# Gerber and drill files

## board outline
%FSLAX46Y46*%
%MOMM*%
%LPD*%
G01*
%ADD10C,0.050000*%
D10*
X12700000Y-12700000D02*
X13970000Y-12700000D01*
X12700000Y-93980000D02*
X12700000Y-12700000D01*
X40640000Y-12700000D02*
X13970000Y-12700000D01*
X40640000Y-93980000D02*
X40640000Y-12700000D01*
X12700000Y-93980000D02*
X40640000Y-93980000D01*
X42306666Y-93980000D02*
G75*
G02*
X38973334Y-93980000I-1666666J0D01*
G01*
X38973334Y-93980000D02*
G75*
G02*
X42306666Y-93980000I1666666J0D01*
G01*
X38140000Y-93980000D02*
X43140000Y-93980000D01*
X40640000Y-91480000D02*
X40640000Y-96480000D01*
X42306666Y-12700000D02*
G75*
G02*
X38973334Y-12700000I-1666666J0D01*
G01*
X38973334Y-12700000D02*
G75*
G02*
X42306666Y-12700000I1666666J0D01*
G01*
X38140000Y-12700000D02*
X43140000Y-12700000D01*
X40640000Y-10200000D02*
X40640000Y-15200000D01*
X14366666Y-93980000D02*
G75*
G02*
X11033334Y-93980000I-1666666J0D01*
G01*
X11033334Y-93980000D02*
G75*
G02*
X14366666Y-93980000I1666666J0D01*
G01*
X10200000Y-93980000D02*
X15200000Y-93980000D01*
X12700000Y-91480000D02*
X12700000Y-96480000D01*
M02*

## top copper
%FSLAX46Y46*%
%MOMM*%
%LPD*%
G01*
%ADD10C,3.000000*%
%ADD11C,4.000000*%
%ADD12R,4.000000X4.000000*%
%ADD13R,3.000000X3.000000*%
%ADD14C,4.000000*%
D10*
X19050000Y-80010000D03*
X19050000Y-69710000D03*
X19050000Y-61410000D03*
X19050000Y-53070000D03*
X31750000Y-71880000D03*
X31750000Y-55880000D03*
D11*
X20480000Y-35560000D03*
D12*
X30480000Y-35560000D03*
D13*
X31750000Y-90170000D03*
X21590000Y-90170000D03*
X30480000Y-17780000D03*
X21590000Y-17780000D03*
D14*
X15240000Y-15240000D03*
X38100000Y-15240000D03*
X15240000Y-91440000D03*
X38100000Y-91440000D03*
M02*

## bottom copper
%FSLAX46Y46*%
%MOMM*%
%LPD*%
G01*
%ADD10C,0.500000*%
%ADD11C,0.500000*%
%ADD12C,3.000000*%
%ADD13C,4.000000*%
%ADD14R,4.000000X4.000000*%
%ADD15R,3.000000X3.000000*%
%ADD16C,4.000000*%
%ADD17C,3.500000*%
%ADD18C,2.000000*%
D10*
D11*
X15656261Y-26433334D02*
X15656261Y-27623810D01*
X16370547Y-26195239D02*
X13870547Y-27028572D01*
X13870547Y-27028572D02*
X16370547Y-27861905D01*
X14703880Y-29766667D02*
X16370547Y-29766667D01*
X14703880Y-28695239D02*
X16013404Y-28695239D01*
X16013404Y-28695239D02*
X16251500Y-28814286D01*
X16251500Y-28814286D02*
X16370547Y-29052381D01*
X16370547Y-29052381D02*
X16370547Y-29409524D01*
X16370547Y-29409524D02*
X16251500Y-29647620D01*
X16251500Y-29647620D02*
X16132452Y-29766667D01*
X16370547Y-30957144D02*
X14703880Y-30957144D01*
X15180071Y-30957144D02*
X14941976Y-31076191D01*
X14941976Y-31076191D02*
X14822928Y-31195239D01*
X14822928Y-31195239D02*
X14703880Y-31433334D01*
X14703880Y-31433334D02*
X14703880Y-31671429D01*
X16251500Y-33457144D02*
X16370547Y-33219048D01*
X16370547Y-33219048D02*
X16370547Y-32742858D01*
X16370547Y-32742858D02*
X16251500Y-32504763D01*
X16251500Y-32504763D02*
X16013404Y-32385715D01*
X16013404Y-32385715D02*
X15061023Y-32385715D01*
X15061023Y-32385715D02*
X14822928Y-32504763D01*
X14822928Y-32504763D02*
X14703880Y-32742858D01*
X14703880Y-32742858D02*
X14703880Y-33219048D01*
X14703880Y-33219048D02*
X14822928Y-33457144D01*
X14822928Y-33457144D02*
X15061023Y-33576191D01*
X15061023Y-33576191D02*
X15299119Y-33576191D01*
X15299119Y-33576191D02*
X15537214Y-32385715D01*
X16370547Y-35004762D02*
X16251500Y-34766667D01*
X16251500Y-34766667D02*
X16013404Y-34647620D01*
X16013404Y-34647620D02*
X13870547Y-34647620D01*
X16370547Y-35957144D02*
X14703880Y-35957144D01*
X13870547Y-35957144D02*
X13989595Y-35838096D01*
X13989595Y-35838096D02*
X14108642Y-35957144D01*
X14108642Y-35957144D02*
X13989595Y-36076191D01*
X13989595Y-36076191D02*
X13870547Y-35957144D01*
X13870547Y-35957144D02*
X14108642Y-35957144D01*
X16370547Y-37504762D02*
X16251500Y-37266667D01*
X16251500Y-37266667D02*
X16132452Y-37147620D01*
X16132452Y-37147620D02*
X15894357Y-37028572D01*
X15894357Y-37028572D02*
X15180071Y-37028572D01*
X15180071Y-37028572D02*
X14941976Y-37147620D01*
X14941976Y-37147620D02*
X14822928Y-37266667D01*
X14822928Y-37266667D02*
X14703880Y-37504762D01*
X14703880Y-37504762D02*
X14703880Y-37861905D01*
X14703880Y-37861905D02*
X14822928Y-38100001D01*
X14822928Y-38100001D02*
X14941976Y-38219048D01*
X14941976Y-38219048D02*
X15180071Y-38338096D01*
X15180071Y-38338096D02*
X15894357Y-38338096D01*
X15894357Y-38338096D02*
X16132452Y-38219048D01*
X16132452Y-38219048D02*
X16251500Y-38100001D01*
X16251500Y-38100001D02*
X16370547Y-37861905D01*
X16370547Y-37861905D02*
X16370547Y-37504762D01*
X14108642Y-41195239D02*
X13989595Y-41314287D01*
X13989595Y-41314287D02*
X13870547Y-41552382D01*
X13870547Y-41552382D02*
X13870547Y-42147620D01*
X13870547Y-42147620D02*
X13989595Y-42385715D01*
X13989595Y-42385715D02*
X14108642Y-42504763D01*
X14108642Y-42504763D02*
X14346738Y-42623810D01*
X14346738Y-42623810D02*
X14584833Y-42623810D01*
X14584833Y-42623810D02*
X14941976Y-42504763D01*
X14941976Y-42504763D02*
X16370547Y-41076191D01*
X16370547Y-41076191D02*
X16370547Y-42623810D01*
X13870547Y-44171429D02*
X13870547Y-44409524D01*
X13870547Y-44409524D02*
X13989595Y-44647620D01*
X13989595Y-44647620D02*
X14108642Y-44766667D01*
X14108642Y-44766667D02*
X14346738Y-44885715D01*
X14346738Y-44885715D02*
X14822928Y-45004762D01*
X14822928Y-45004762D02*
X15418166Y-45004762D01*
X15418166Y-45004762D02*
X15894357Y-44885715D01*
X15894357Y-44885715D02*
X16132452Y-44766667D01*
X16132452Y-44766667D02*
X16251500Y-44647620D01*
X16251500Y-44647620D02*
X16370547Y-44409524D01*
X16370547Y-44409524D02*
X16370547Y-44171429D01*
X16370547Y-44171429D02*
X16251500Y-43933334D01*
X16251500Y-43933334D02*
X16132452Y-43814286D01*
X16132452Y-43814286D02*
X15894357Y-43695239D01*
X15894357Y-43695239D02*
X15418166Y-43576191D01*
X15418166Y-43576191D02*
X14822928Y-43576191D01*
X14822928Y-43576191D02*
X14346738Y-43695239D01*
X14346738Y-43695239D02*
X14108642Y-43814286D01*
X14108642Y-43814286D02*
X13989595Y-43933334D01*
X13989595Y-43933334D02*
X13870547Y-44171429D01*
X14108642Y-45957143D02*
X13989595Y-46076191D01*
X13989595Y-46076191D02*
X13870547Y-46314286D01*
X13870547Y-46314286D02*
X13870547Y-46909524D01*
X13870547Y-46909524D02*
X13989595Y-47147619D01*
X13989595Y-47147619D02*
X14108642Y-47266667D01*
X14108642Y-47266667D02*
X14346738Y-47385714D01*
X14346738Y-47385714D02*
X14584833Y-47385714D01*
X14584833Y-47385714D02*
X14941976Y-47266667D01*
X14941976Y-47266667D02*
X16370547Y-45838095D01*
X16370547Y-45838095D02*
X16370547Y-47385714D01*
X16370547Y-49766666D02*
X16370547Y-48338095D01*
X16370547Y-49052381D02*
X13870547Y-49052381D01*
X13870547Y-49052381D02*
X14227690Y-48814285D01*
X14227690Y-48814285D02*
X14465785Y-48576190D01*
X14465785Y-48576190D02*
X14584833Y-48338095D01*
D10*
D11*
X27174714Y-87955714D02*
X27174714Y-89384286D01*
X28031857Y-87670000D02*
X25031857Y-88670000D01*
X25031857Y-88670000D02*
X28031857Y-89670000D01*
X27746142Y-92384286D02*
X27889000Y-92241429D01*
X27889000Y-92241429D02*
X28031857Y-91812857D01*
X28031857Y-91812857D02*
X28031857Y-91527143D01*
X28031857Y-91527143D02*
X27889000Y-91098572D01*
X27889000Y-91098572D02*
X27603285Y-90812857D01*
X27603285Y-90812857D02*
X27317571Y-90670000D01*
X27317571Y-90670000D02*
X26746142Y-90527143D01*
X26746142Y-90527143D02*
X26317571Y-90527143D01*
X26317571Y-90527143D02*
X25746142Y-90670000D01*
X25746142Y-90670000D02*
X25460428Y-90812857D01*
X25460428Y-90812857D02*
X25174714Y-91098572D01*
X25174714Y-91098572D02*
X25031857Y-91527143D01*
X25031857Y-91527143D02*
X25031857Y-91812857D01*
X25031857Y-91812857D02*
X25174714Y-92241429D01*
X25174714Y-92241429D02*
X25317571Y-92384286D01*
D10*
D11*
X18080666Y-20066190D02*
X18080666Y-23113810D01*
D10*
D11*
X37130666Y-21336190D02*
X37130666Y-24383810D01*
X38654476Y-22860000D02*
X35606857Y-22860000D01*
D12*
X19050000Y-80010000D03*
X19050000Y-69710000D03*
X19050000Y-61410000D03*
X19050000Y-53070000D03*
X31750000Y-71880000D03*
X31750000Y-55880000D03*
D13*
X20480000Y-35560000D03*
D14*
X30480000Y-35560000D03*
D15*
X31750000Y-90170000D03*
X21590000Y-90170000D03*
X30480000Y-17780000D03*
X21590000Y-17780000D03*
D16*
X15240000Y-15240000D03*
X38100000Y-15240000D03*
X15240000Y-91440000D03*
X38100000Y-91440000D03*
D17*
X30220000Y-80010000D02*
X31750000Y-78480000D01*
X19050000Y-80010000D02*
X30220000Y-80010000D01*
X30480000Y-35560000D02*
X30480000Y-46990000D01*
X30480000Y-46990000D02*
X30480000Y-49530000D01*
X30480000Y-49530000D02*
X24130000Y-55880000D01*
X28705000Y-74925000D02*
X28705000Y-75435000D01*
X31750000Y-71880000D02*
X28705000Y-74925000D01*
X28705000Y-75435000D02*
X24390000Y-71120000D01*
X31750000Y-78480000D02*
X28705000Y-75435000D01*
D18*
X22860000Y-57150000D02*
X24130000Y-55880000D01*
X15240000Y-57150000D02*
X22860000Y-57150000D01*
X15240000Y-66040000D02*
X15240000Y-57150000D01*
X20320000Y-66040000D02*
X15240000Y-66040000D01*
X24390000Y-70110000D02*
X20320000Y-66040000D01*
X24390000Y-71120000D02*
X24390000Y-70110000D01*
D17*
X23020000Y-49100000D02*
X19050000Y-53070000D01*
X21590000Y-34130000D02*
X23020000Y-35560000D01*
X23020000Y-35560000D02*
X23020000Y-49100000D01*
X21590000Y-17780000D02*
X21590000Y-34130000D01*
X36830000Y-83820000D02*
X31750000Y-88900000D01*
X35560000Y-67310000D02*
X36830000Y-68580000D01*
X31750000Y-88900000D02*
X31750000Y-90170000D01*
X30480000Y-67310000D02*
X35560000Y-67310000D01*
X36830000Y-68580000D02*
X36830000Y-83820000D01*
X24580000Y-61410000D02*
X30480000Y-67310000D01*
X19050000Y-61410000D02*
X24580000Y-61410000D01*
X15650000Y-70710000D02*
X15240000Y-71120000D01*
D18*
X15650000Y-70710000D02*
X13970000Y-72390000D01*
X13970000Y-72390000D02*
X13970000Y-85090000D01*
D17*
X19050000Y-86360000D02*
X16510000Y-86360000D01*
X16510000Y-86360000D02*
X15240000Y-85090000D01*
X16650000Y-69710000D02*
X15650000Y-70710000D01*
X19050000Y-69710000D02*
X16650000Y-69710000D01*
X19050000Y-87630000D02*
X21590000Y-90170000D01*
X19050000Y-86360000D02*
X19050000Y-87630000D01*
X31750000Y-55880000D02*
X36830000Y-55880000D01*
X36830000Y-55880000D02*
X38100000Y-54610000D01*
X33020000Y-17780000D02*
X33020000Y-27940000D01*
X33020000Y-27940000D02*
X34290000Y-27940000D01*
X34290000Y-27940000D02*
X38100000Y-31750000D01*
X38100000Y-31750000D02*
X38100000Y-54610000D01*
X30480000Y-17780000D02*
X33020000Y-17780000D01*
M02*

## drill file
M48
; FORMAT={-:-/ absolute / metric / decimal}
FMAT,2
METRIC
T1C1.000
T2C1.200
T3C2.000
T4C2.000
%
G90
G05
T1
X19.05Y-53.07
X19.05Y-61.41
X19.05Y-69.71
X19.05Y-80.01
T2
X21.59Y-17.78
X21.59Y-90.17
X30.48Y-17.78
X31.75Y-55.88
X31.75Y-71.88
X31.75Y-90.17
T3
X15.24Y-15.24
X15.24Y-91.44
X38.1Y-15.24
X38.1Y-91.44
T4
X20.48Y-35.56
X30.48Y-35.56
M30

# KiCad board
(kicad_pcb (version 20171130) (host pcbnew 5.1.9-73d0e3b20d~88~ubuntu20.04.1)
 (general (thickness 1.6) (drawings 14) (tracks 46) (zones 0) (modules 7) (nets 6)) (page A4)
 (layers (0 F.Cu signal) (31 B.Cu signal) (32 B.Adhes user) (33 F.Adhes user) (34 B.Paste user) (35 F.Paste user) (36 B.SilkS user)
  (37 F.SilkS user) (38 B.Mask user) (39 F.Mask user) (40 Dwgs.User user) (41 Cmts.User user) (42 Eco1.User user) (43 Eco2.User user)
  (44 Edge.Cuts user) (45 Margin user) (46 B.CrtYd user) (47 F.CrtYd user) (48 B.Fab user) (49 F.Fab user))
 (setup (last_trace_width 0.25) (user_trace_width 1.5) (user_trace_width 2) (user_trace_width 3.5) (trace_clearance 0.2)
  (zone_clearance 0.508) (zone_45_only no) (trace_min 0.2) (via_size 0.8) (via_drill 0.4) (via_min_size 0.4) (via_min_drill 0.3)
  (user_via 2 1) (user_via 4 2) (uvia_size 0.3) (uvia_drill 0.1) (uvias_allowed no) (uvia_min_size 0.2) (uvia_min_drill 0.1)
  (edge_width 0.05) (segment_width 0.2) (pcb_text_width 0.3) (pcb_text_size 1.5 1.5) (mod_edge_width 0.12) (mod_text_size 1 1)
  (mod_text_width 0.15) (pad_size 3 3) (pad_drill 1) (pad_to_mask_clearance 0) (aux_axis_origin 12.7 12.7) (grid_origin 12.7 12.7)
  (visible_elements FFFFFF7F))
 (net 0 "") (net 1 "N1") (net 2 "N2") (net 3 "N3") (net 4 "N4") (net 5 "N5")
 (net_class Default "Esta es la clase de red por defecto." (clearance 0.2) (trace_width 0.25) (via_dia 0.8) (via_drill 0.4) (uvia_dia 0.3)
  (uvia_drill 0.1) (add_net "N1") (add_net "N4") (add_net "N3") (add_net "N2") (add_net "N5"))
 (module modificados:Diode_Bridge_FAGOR (layer F.Cu) (at 19.05 78.74 90)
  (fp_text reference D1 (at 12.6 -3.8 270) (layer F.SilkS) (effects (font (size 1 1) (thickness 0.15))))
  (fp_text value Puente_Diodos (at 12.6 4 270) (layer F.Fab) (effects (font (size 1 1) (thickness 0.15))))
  (pad 1 thru_hole circle (at -1.27 0 90) (size 3 3) (drill 1) (layers *.Cu *.Mask) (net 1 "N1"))
  (pad 4 thru_hole circle (at 9.03 0 90) (size 3 3) (drill 1) (layers *.Cu *.Mask) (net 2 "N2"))
  (pad 3 thru_hole circle (at 17.33 0 90) (size 3 3) (drill 1) (layers *.Cu *.Mask) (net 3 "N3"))
  (pad 2 thru_hole circle (at 25.67 0 90) (size 3 3) (drill 1) (layers *.Cu *.Mask) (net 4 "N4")))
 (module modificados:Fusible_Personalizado (layer F.Cu) (at 31.75 55.88 270)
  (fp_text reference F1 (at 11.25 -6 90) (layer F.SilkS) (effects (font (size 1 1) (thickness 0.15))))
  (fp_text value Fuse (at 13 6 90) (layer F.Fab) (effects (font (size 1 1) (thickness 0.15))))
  (pad 2 thru_hole circle (at 16 0 270) (size 3 3) (drill 1.2) (layers *.Cu *.Mask) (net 1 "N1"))
  (pad 1 thru_hole circle (at 0 0 270) (size 3 3) (drill 1.2) (layers *.Cu *.Mask) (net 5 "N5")))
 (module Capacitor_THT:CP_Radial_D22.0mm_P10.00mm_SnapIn (layer F.Cu) (at 30.48 35.56 180)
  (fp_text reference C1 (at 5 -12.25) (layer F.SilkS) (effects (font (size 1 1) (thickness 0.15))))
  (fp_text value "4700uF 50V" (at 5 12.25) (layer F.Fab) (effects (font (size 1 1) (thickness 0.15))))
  (pad 2 thru_hole circle (at 10 0 180) (size 4 4) (drill 2) (layers *.Cu *.Mask) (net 4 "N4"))
  (pad 1 thru_hole rect (at 0 0 180) (size 4 4) (drill 2) (layers *.Cu *.Mask) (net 1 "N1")))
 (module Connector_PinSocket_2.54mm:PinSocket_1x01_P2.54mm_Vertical (layer F.Cu) (at 31.75 90.17 90)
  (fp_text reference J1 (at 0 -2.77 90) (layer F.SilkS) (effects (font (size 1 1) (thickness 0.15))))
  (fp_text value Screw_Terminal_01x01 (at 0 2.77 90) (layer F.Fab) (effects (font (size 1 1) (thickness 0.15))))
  (pad 1 thru_hole rect (at 0 0 90) (size 3 3) (drill 1.2) (layers *.Cu *.Mask) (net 3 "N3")))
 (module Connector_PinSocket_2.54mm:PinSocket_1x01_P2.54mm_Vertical (layer F.Cu) (at 21.59 90.17 90)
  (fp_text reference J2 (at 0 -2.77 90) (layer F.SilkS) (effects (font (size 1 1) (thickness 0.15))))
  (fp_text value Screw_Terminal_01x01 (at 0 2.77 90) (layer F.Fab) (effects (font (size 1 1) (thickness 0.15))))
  (pad 1 thru_hole rect (at 0 0 90) (size 3 3) (drill 1.2) (layers *.Cu *.Mask) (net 2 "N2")))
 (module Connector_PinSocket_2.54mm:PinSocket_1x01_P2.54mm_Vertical (layer F.Cu) (at 30.48 17.78 90)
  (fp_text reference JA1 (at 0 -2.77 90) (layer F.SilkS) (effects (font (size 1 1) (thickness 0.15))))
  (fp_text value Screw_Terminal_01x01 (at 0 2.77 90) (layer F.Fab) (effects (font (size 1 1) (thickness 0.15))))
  (pad 1 thru_hole rect (at 0 0 90) (size 3 3) (drill 1.2) (layers *.Cu *.Mask) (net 5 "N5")))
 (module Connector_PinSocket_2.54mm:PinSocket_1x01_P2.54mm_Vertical (layer F.Cu) (at 21.59 17.78 90)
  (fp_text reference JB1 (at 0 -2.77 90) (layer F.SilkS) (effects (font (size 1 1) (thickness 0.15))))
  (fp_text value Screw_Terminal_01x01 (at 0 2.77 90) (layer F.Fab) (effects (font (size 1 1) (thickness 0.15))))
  (pad 1 thru_hole rect (at 0 0 90) (size 3 3) (drill 1.2) (layers *.Cu *.Mask) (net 4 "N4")))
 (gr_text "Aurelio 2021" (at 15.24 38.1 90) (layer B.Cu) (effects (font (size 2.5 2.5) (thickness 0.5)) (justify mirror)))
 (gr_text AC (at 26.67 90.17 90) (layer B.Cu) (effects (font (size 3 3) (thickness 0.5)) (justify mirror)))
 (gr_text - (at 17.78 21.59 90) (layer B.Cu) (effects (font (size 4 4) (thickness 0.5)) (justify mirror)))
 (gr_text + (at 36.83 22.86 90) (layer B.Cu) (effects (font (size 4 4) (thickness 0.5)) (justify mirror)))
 (gr_line (start 12.7 12.7) (end 13.97 12.7) (layer Edge.Cuts) (width 0.05))
 (gr_line (start 12.7 93.98) (end 12.7 12.7) (layer Edge.Cuts) (width 0.05))
 (gr_line (start 40.64 12.7) (end 13.97 12.7) (layer Edge.Cuts) (width 0.05))
 (gr_line (start 40.64 93.98) (end 40.64 12.7) (layer Edge.Cuts) (width 0.05))
 (gr_line (start 12.7 93.98) (end 40.64 93.98) (layer Edge.Cuts) (width 0.05))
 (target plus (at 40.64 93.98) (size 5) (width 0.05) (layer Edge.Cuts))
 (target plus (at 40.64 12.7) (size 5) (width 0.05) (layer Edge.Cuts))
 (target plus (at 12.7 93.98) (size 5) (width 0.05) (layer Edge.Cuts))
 (via (at 15.24 15.24) (size 4) (drill 2) (layers F.Cu B.Cu) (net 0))
 (via (at 38.1 15.24) (size 4) (drill 2) (layers F.Cu B.Cu) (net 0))
 (via (at 15.24 91.44) (size 4) (drill 2) (layers F.Cu B.Cu) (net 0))
 (via (at 38.1 91.44) (size 4) (drill 2) (layers F.Cu B.Cu) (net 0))
 (segment (start 30.22 80.01) (end 31.75 78.48) (width 3.5) (layer B.Cu) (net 1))
 (segment (start 19.05 80.01) (end 30.22 80.01) (width 3.5) (layer B.Cu) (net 1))
 (segment (start 30.48 35.56) (end 30.48 46.99) (width 3.5) (layer B.Cu) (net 1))
 (segment (start 30.48 46.99) (end 30.48 49.53) (width 3.5) (layer B.Cu) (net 1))
 (segment (start 30.48 49.53) (end 24.13 55.88) (width 3.5) (layer B.Cu) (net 1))
 (segment (start 28.705 74.925) (end 28.705 75.435) (width 3.5) (layer B.Cu) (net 1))
 (segment (start 31.75 71.88) (end 28.705 74.925) (width 3.5) (layer B.Cu) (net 1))
 (segment (start 28.705 75.435) (end 24.39 71.12) (width 3.5) (layer B.Cu) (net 1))
 (segment (start 31.75 78.48) (end 28.705 75.435) (width 3.5) (layer B.Cu) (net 1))
 (segment (start 22.86 57.15) (end 24.13 55.88) (width 2) (layer B.Cu) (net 1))
 (segment (start 15.24 57.15) (end 22.86 57.15) (width 2) (layer B.Cu) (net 1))
 (segment (start 15.24 66.04) (end 15.24 57.15) (width 2) (layer B.Cu) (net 1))
 (segment (start 20.32 66.04) (end 15.24 66.04) (width 2) (layer B.Cu) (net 1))
 (segment (start 24.39 70.11) (end 20.32 66.04) (width 2) (layer B.Cu) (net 1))
 (segment (start 24.39 71.12) (end 24.39 70.11) (width 2) (layer B.Cu) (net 1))
 (segment (start 23.02 49.1) (end 19.05 53.07) (width 3.5) (layer B.Cu) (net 4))
 (segment (start 21.59 34.13) (end 23.02 35.56) (width 3.5) (layer B.Cu) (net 4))
 (segment (start 23.02 35.56) (end 23.02 49.1) (width 3.5) (layer B.Cu) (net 4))
 (segment (start 21.59 17.78) (end 21.59 34.13) (width 3.5) (layer B.Cu) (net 4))
 (segment (start 36.83 83.82) (end 31.75 88.9) (width 3.5) (layer B.Cu) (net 3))
 (segment (start 35.56 67.31) (end 36.83 68.58) (width 3.5) (layer B.Cu) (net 3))
 (segment (start 31.75 88.9) (end 31.75 90.17) (width 3.5) (layer B.Cu) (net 3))
 (segment (start 30.48 67.31) (end 35.56 67.31) (width 3.5) (layer B.Cu) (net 3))
 (segment (start 36.83 68.58) (end 36.83 83.82) (width 3.5) (layer B.Cu) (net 3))
 (segment (start 24.58 61.41) (end 30.48 67.31) (width 3.5) (layer B.Cu) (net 3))
 (segment (start 19.05 61.41) (end 24.58 61.41) (width 3.5) (layer B.Cu) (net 3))
 (segment (start 15.65 70.71) (end 15.24 71.12) (width 3.5) (layer B.Cu) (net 2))
 (segment (start 15.65 70.71) (end 13.97 72.39) (width 2) (layer B.Cu) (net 2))
 (segment (start 13.97 72.39) (end 13.97 85.09) (width 2) (layer B.Cu) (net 2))
 (segment (start 19.05 86.36) (end 16.51 86.36) (width 3.5) (layer B.Cu) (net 2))
 (segment (start 16.51 86.36) (end 15.24 85.09) (width 3.5) (layer B.Cu) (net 2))
 (segment (start 16.65 69.71) (end 15.65 70.71) (width 3.5) (layer B.Cu) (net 2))
 (segment (start 19.05 69.71) (end 16.65 69.71) (width 3.5) (layer B.Cu) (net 2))
 (segment (start 19.05 87.63) (end 21.59 90.17) (width 3.5) (layer B.Cu) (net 2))
 (segment (start 19.05 86.36) (end 19.05 87.63) (width 3.5) (layer B.Cu) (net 2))
 (segment (start 31.75 55.88) (end 36.83 55.88) (width 3.5) (layer B.Cu) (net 5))
 (segment (start 36.83 55.88) (end 38.1 54.61) (width 3.5) (layer B.Cu) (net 5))
 (segment (start 33.02 17.78) (end 33.02 27.94) (width 3.5) (layer B.Cu) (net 5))
 (segment (start 33.02 27.94) (end 34.29 27.94) (width 3.5) (layer B.Cu) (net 5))
 (segment (start 34.29 27.94) (end 38.1 31.75) (width 3.5) (layer B.Cu) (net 5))
 (segment (start 38.1 31.75) (end 38.1 54.61) (width 3.5) (layer B.Cu) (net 5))
 (segment (start 30.48 17.78) (end 33.02 17.78) (width 3.5) (layer B.Cu) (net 5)))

